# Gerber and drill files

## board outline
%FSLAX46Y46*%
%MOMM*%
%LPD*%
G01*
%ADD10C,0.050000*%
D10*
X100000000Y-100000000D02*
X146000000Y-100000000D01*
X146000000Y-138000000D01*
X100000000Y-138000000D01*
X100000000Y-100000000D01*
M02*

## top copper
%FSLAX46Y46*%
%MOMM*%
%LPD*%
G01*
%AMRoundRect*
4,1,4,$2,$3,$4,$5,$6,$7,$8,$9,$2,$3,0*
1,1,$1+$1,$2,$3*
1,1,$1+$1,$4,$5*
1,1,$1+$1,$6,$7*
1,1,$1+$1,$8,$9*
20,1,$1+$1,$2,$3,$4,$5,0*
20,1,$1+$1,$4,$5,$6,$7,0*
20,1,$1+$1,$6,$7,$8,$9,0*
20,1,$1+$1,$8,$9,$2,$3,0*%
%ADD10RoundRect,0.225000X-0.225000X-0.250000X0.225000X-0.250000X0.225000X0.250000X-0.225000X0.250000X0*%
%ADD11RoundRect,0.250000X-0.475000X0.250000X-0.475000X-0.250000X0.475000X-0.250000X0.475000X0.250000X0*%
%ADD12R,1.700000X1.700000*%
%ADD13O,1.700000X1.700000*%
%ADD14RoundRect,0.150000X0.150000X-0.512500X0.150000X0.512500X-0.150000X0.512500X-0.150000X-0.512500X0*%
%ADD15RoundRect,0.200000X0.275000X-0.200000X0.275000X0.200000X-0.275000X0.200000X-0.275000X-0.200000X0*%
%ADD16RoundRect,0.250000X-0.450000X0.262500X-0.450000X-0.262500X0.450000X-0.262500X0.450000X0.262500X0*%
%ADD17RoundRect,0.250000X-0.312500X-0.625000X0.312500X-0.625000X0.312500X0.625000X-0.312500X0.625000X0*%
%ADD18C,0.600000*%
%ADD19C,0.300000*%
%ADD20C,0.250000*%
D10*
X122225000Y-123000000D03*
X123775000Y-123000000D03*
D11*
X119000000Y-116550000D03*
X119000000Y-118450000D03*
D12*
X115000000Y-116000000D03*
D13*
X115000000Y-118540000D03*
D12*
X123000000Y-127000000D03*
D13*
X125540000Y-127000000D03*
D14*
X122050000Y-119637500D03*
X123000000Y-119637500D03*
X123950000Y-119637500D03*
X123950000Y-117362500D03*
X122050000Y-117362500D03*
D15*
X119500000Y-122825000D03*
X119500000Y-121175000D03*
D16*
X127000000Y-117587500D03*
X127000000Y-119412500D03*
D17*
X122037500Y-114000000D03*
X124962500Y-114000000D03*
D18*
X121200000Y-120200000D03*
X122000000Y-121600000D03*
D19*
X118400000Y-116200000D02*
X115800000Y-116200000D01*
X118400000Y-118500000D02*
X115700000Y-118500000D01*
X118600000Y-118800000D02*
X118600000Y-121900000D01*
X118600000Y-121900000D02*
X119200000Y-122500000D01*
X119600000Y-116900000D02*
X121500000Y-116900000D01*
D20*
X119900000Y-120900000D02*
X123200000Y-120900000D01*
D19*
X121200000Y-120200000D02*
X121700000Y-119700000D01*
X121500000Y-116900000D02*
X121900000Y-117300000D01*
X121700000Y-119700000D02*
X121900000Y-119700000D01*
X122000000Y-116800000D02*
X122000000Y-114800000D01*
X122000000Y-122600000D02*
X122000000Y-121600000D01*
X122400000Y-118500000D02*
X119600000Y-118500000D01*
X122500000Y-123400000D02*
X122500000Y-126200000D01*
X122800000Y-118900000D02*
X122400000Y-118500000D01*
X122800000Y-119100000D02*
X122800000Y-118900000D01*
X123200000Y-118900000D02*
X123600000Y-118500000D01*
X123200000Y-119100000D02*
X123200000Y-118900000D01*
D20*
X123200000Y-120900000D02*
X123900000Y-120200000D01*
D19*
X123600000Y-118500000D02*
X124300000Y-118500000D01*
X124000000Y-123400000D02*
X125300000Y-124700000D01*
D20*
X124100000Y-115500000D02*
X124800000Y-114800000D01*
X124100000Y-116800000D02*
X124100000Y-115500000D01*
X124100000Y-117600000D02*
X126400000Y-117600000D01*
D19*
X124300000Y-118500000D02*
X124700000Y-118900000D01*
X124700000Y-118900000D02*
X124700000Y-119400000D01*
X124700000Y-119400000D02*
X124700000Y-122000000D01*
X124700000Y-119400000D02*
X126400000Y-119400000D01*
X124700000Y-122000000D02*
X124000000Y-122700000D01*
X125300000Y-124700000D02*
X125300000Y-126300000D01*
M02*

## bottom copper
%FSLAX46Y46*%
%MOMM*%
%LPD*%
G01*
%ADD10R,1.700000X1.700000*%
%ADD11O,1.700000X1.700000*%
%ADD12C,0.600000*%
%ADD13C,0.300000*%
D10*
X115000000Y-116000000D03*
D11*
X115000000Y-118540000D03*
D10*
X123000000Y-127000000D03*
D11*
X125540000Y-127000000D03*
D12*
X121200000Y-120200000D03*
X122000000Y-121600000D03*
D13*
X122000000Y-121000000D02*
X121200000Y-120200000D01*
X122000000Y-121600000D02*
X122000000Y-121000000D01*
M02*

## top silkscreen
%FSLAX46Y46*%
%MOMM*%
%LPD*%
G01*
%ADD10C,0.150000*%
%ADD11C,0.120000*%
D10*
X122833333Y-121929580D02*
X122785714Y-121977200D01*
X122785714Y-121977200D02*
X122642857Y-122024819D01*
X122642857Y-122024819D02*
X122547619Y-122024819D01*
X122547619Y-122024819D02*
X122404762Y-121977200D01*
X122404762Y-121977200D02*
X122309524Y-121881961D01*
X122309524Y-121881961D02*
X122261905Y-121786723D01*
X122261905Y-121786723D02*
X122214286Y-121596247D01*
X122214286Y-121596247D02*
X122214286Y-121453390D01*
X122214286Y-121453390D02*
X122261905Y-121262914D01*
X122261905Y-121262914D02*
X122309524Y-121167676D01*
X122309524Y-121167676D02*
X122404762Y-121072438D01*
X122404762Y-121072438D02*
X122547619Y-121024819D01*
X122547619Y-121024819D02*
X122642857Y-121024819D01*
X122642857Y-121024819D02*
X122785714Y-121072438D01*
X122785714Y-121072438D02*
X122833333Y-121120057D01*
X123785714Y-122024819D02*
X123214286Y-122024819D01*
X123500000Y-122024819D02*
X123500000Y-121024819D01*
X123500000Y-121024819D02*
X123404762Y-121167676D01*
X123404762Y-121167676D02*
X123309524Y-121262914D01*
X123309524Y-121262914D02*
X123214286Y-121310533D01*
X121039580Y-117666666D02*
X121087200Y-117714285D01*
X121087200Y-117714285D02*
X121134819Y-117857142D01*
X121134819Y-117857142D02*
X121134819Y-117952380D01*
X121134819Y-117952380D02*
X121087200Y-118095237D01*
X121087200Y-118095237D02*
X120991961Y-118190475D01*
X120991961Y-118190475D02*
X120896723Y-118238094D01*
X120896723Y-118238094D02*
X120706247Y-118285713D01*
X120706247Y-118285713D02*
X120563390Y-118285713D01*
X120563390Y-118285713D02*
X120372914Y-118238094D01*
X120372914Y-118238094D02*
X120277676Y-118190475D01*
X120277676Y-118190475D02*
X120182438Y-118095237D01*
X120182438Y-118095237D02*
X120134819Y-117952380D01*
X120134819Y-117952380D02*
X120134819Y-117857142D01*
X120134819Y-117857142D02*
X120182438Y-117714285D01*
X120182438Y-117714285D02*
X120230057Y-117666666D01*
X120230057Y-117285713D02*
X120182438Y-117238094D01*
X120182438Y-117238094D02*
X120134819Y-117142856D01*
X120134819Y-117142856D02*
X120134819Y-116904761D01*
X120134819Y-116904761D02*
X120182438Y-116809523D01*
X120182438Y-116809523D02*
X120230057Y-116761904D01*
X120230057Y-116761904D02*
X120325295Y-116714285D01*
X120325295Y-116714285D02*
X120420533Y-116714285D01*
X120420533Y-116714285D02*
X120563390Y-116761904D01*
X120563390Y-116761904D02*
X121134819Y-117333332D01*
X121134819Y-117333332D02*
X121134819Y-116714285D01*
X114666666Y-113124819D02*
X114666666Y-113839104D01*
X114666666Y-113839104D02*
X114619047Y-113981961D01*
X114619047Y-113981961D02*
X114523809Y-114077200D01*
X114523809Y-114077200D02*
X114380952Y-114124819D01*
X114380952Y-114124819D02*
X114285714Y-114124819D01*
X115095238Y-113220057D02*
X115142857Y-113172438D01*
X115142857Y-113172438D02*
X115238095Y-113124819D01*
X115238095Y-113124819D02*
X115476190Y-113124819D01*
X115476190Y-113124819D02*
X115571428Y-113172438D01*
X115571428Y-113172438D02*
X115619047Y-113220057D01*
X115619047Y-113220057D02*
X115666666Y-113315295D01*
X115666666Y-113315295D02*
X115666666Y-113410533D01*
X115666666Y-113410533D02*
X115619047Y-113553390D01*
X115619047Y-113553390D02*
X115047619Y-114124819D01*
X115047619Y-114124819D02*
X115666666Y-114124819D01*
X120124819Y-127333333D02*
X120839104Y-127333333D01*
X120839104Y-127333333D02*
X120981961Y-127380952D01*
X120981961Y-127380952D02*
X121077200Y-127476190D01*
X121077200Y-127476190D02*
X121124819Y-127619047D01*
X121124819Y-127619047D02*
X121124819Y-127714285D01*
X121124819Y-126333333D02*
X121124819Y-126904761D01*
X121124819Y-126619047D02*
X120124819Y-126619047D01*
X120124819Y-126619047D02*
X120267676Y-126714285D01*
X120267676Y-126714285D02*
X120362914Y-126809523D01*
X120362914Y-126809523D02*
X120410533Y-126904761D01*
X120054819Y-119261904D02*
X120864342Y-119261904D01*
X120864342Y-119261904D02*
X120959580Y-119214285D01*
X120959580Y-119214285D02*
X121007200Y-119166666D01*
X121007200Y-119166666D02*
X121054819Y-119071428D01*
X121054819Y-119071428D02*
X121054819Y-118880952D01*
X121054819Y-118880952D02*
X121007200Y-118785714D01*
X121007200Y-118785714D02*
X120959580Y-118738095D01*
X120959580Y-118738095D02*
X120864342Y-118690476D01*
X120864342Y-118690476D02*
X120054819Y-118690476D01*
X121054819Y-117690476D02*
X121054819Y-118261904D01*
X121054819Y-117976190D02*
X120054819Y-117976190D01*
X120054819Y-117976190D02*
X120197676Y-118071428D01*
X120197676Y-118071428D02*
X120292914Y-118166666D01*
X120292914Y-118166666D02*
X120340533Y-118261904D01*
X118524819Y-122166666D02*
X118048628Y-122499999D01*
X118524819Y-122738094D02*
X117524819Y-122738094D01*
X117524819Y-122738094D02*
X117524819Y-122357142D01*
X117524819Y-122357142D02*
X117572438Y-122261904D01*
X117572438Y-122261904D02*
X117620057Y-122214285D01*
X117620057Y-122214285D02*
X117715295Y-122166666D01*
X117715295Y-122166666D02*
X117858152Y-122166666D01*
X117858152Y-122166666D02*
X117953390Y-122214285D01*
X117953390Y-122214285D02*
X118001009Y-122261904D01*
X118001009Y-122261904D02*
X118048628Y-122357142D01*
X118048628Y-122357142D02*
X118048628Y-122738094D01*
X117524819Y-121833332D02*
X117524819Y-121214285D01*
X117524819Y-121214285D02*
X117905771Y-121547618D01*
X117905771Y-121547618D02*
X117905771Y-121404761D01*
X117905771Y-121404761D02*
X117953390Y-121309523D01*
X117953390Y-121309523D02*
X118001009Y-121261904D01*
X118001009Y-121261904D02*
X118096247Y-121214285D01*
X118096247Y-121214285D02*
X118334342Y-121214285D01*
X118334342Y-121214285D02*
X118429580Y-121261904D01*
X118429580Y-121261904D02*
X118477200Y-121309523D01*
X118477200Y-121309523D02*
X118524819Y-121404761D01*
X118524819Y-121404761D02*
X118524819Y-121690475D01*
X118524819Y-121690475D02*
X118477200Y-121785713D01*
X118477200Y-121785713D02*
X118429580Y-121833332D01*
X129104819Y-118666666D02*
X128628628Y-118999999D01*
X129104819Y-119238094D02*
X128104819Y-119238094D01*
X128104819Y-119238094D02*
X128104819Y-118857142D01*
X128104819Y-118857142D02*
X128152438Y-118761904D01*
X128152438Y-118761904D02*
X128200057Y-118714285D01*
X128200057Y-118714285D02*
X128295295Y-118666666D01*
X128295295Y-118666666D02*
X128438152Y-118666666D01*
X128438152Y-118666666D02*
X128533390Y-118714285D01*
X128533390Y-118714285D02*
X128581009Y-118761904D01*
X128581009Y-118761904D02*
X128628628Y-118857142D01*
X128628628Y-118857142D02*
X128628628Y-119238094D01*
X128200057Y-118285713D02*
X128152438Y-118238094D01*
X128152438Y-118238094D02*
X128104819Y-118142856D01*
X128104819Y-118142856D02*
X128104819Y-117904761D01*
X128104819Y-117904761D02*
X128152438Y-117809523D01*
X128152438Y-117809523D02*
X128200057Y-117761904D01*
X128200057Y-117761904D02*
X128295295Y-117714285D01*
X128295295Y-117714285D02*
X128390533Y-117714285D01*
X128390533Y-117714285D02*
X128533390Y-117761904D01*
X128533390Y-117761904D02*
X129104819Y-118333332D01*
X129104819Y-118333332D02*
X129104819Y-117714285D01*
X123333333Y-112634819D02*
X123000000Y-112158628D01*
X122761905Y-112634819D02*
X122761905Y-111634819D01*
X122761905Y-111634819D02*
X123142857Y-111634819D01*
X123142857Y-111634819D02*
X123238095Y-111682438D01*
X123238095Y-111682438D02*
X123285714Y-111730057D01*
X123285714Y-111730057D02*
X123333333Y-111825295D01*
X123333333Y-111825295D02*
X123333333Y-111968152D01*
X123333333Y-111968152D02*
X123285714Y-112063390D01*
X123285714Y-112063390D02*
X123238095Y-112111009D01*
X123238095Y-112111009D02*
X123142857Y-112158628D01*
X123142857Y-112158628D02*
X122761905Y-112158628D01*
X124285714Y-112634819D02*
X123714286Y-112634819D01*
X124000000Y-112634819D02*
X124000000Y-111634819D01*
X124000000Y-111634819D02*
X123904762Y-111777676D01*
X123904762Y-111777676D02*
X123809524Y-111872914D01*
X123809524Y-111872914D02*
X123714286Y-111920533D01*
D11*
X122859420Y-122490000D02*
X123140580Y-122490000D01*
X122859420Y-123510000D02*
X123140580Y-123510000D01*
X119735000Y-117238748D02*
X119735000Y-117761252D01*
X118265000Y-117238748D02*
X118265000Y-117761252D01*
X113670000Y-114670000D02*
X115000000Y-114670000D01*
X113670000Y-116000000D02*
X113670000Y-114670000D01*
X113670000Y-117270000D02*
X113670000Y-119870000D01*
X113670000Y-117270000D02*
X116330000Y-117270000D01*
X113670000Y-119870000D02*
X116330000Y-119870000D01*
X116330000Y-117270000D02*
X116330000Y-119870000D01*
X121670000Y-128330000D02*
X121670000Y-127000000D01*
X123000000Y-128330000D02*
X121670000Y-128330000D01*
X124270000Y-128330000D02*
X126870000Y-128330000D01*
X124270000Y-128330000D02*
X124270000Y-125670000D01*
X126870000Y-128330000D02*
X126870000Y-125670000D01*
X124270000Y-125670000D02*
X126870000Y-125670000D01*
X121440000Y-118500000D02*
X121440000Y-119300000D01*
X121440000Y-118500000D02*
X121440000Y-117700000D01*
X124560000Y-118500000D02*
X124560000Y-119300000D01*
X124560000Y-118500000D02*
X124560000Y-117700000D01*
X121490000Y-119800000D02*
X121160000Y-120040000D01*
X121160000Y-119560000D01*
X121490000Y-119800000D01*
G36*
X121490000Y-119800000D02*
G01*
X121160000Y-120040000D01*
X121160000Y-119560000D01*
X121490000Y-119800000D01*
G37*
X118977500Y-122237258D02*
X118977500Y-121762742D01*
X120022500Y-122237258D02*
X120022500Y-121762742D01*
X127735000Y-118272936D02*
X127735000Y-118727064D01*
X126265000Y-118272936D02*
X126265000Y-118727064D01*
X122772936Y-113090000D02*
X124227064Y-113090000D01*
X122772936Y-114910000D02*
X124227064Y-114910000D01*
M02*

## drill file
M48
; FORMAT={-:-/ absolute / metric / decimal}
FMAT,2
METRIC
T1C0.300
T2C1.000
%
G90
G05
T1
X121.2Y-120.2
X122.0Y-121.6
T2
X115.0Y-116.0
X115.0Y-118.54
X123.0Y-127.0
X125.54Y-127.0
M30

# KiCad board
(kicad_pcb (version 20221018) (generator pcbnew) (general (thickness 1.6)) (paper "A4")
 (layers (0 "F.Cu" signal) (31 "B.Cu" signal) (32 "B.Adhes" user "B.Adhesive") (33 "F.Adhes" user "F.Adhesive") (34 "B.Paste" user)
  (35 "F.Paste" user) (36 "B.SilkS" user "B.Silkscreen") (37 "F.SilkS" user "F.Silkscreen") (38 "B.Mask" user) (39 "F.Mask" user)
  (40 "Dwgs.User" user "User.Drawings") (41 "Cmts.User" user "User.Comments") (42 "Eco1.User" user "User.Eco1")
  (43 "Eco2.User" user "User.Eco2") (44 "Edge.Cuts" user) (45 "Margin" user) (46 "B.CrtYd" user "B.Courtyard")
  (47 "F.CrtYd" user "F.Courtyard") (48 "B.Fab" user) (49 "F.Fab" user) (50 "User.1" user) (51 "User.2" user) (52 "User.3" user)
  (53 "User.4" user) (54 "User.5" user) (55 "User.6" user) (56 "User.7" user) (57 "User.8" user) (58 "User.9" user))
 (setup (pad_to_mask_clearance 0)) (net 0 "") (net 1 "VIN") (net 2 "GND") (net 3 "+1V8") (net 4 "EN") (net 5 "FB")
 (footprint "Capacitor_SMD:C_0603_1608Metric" (layer "F.Cu") (at 123 123)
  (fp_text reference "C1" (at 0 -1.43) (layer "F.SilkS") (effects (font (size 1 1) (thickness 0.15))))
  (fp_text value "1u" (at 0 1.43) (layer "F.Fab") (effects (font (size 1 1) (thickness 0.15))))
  (fp_line (start -0.14058 -0.51) (end 0.14058 -0.51) (stroke (width 0.12) (type solid)) (layer "F.SilkS"))
  (fp_line (start -0.14058 0.51) (end 0.14058 0.51) (stroke (width 0.12) (type solid)) (layer "F.SilkS"))
  (pad "1" smd roundrect (at -0.775 0) (size 0.9 0.95) (layers "F.Cu" "F.Paste" "F.Mask") (roundrect_rratio 0.25) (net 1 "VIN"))
  (pad "2" smd roundrect (at 0.775 0) (size 0.9 0.95) (layers "F.Cu" "F.Paste" "F.Mask") (roundrect_rratio 0.25) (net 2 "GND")))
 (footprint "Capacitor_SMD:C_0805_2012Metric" (layer "F.Cu") (at 119 117.5 -90)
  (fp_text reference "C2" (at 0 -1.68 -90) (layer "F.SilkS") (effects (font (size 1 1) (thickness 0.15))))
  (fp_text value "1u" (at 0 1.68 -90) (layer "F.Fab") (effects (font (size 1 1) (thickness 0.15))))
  (fp_line (start -0.261252 -0.735) (end 0.261252 -0.735) (stroke (width 0.12) (type solid)) (layer "F.SilkS"))
  (fp_line (start -0.261252 0.735) (end 0.261252 0.735) (stroke (width 0.12) (type solid)) (layer "F.SilkS"))
  (pad "1" smd roundrect (at -0.95 0 270) (size 1 1.45) (layers "F.Cu" "F.Paste" "F.Mask") (roundrect_rratio 0.25) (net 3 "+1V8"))
  (pad "2" smd roundrect (at 0.95 0 270) (size 1 1.45) (layers "F.Cu" "F.Paste" "F.Mask") (roundrect_rratio 0.25) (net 2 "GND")))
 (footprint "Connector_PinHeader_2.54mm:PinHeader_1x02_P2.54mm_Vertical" (layer "F.Cu") (at 115 116)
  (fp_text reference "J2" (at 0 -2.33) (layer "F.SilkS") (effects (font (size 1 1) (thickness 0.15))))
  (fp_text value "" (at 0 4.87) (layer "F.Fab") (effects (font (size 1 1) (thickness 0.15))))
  (fp_line (start -1.33 -1.33) (end 0 -1.33) (stroke (width 0.12) (type solid)) (layer "F.SilkS"))
  (fp_line (start -1.33 0) (end -1.33 -1.33) (stroke (width 0.12) (type solid)) (layer "F.SilkS"))
  (fp_line (start -1.33 1.27) (end -1.33 3.87) (stroke (width 0.12) (type solid)) (layer "F.SilkS"))
  (fp_line (start -1.33 1.27) (end 1.33 1.27) (stroke (width 0.12) (type solid)) (layer "F.SilkS"))
  (fp_line (start -1.33 3.87) (end 1.33 3.87) (stroke (width 0.12) (type solid)) (layer "F.SilkS"))
  (fp_line (start 1.33 1.27) (end 1.33 3.87) (stroke (width 0.12) (type solid)) (layer "F.SilkS"))
  (pad "1" thru_hole rect (at 0 0) (size 1.7 1.7) (drill 1) (layers "*.Cu" "*.Mask") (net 3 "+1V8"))
  (pad "2" thru_hole oval (at 0 2.54) (size 1.7 1.7) (drill 1) (layers "*.Cu" "*.Mask") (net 2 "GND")))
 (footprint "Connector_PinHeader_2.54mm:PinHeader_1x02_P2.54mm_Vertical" (layer "F.Cu") (at 123 127 90)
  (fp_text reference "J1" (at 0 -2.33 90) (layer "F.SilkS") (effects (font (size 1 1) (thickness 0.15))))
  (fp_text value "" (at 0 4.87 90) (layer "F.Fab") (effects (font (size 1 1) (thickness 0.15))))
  (fp_line (start -1.33 -1.33) (end 0 -1.33) (stroke (width 0.12) (type solid)) (layer "F.SilkS"))
  (fp_line (start -1.33 0) (end -1.33 -1.33) (stroke (width 0.12) (type solid)) (layer "F.SilkS"))
  (fp_line (start -1.33 1.27) (end -1.33 3.87) (stroke (width 0.12) (type solid)) (layer "F.SilkS"))
  (fp_line (start -1.33 1.27) (end 1.33 1.27) (stroke (width 0.12) (type solid)) (layer "F.SilkS"))
  (fp_line (start -1.33 3.87) (end 1.33 3.87) (stroke (width 0.12) (type solid)) (layer "F.SilkS"))
  (fp_line (start 1.33 1.27) (end 1.33 3.87) (stroke (width 0.12) (type solid)) (layer "F.SilkS"))
  (pad "1" thru_hole rect (at 0 0 90) (size 1.7 1.7) (drill 1) (layers "*.Cu" "*.Mask") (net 1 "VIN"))
  (pad "2" thru_hole oval (at 0 2.54 90) (size 1.7 1.7) (drill 1) (layers "*.Cu" "*.Mask") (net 2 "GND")))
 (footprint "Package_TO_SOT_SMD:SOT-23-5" (layer "F.Cu") (at 123 118.5 90)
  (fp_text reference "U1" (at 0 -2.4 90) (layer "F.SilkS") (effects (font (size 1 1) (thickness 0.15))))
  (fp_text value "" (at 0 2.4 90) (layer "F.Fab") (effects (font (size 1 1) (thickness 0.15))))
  (fp_line (start 0 -1.56) (end -0.8 -1.56) (stroke (width 0.12) (type solid)) (layer "F.SilkS"))
  (fp_line (start 0 -1.56) (end 0.8 -1.56) (stroke (width 0.12) (type solid)) (layer "F.SilkS"))
  (fp_line (start 0 1.56) (end -0.8 1.56) (stroke (width 0.12) (type solid)) (layer "F.SilkS"))
  (fp_line (start 0 1.56) (end 0.8 1.56) (stroke (width 0.12) (type solid)) (layer "F.SilkS"))
  (fp_poly
   (pts (xy -1.3 -1.51) (xy -1.54 -1.84) (xy -1.06 -1.84) (xy -1.3 -1.51)) (stroke (width 0.12) (type solid)) (fill solid) (layer "F.SilkS"))
  (pad "1" smd roundrect (at -1.1375 -0.95 90) (size 1.325 0.6) (layers "F.Cu" "F.Paste" "F.Mask") (roundrect_rratio 0.25) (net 1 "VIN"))
  (pad "2" smd roundrect (at -1.1375 0 90) (size 1.325 0.6) (layers "F.Cu" "F.Paste" "F.Mask") (roundrect_rratio 0.25) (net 2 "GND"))
  (pad "3" smd roundrect (at -1.1375 0.95 90) (size 1.325 0.6) (layers "F.Cu" "F.Paste" "F.Mask") (roundrect_rratio 0.25) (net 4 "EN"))
  (pad "4" smd roundrect (at 1.1375 0.95 90) (size 1.325 0.6) (layers "F.Cu" "F.Paste" "F.Mask") (roundrect_rratio 0.25) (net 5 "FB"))
  (pad "5" smd roundrect (at 1.1375 -0.95 90) (size 1.325 0.6) (layers "F.Cu" "F.Paste" "F.Mask") (roundrect_rratio 0.25) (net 3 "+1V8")))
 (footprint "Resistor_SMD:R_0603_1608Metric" (layer "F.Cu") (at 119.5 122 90)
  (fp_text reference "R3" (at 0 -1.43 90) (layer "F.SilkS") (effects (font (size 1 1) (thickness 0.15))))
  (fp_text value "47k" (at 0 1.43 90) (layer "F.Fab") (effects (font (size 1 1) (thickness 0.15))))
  (fp_line (start -0.237258 -0.5225) (end 0.237258 -0.5225) (stroke (width 0.12) (type solid)) (layer "F.SilkS"))
  (fp_line (start -0.237258 0.5225) (end 0.237258 0.5225) (stroke (width 0.12) (type solid)) (layer "F.SilkS"))
  (pad "1" smd roundrect (at -0.825 0 90) (size 0.8 0.95) (layers "F.Cu" "F.Paste" "F.Mask") (roundrect_rratio 0.25) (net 2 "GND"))
  (pad "2" smd roundrect (at 0.825 0 90) (size 0.8 0.95) (layers "F.Cu" "F.Paste" "F.Mask") (roundrect_rratio 0.25) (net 4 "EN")))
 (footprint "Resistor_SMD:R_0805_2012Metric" (layer "F.Cu") (at 127 118.5 -90)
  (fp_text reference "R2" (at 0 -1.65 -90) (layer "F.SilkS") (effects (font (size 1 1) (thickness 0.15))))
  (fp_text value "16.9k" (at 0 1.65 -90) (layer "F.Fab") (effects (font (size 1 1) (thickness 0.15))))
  (fp_line (start -0.227064 -0.735) (end 0.227064 -0.735) (stroke (width 0.12) (type solid)) (layer "F.SilkS"))
  (fp_line (start -0.227064 0.735) (end 0.227064 0.735) (stroke (width 0.12) (type solid)) (layer "F.SilkS"))
  (pad "1" smd roundrect (at -0.9125 0 270) (size 1.025 1.4) (layers "F.Cu" "F.Paste" "F.Mask") (roundrect_rratio 0.243902) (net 5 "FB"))
  (pad "2" smd roundrect (at 0.9125 0 270) (size 1.025 1.4) (layers "F.Cu" "F.Paste" "F.Mask") (roundrect_rratio 0.243902) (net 2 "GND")))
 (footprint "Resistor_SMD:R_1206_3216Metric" (layer "F.Cu") (at 123.5 114)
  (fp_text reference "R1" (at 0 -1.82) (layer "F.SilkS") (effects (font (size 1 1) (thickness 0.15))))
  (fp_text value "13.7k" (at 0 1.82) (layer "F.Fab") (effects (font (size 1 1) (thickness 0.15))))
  (fp_line (start -0.727064 -0.91) (end 0.727064 -0.91) (stroke (width 0.12) (type solid)) (layer "F.SilkS"))
  (fp_line (start -0.727064 0.91) (end 0.727064 0.91) (stroke (width 0.12) (type solid)) (layer "F.SilkS"))
  (pad "1" smd roundrect (at -1.4625 0) (size 1.125 1.75) (layers "F.Cu" "F.Paste" "F.Mask") (roundrect_rratio 0.222222) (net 3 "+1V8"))
  (pad "2" smd roundrect (at 1.4625 0) (size 1.125 1.75) (layers "F.Cu" "F.Paste" "F.Mask") (roundrect_rratio 0.222222) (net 5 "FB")))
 (gr_rect (start 100 100) (end 146 138) (stroke (width 0.05) (type default)) (fill none) (layer "Edge.Cuts"))
 (segment (start 118.4 116.2) (end 115.8 116.2) (width 0.3) (layer "F.Cu") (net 3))
 (segment (start 118.4 118.5) (end 115.7 118.5) (width 0.3) (layer "F.Cu") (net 2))
 (segment (start 118.6 118.8) (end 118.6 121.9) (width 0.3) (layer "F.Cu") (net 2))
 (segment (start 118.6 121.9) (end 119.2 122.5) (width 0.3) (layer "F.Cu") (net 2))
 (segment (start 119.6 116.9) (end 121.5 116.9) (width 0.3) (layer "F.Cu") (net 3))
 (segment (start 119.9 120.9) (end 123.2 120.9) (width 0.25) (layer "F.Cu") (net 4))
 (segment (start 121.2 120.2) (end 121.7 119.7) (width 0.3) (layer "F.Cu") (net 1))
 (segment (start 121.5 116.9) (end 121.9 117.3) (width 0.3) (layer "F.Cu") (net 3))
 (segment (start 121.7 119.7) (end 121.9 119.7) (width 0.3) (layer "F.Cu") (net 1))
 (segment (start 122 116.8) (end 122 114.8) (width 0.3) (layer "F.Cu") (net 3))
 (segment (start 122 122.6) (end 122 121.6) (width 0.3) (layer "F.Cu") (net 1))
 (segment (start 122.4 118.5) (end 119.6 118.5) (width 0.3) (layer "F.Cu") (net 2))
 (segment (start 122.5 123.4) (end 122.5 126.2) (width 0.3) (layer "F.Cu") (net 1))
 (segment (start 122.8 118.9) (end 122.4 118.5) (width 0.3) (layer "F.Cu") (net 2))
 (segment (start 122.8 119.1) (end 122.8 118.9) (width 0.3) (layer "F.Cu") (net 2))
 (segment (start 123.2 118.9) (end 123.6 118.5) (width 0.3) (layer "F.Cu") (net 2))
 (segment (start 123.2 119.1) (end 123.2 118.9) (width 0.3) (layer "F.Cu") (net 2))
 (segment (start 123.2 120.9) (end 123.9 120.2) (width 0.25) (layer "F.Cu") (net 4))
 (segment (start 123.6 118.5) (end 124.3 118.5) (width 0.3) (layer "F.Cu") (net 2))
 (segment (start 124 123.4) (end 125.3 124.7) (width 0.3) (layer "F.Cu") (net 2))
 (segment (start 124.1 115.5) (end 124.8 114.8) (width 0.25) (layer "F.Cu") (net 5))
 (segment (start 124.1 116.8) (end 124.1 115.5) (width 0.25) (layer "F.Cu") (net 5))
 (segment (start 124.1 117.6) (end 126.4 117.6) (width 0.25) (layer "F.Cu") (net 5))
 (segment (start 124.3 118.5) (end 124.7 118.9) (width 0.3) (layer "F.Cu") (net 2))
 (segment (start 124.7 118.9) (end 124.7 119.4) (width 0.3) (layer "F.Cu") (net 2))
 (segment (start 124.7 119.4) (end 124.7 122) (width 0.3) (layer "F.Cu") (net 2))
 (segment (start 124.7 119.4) (end 126.4 119.4) (width 0.3) (layer "F.Cu") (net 2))
 (segment (start 124.7 122) (end 124 122.7) (width 0.3) (layer "F.Cu") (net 2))
 (segment (start 125.3 124.7) (end 125.3 126.3) (width 0.3) (layer "F.Cu") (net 2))
 (via (at 121.2 120.2) (size 0.6) (drill 0.3) (layers "F.Cu" "B.Cu") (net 1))
 (via (at 122 121.6) (size 0.6) (drill 0.3) (layers "F.Cu" "B.Cu") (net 1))
 (segment (start 122 121) (end 121.2 120.2) (width 0.3) (layer "B.Cu") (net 1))
 (segment (start 122 121.6) (end 122 121) (width 0.3) (layer "B.Cu") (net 1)))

